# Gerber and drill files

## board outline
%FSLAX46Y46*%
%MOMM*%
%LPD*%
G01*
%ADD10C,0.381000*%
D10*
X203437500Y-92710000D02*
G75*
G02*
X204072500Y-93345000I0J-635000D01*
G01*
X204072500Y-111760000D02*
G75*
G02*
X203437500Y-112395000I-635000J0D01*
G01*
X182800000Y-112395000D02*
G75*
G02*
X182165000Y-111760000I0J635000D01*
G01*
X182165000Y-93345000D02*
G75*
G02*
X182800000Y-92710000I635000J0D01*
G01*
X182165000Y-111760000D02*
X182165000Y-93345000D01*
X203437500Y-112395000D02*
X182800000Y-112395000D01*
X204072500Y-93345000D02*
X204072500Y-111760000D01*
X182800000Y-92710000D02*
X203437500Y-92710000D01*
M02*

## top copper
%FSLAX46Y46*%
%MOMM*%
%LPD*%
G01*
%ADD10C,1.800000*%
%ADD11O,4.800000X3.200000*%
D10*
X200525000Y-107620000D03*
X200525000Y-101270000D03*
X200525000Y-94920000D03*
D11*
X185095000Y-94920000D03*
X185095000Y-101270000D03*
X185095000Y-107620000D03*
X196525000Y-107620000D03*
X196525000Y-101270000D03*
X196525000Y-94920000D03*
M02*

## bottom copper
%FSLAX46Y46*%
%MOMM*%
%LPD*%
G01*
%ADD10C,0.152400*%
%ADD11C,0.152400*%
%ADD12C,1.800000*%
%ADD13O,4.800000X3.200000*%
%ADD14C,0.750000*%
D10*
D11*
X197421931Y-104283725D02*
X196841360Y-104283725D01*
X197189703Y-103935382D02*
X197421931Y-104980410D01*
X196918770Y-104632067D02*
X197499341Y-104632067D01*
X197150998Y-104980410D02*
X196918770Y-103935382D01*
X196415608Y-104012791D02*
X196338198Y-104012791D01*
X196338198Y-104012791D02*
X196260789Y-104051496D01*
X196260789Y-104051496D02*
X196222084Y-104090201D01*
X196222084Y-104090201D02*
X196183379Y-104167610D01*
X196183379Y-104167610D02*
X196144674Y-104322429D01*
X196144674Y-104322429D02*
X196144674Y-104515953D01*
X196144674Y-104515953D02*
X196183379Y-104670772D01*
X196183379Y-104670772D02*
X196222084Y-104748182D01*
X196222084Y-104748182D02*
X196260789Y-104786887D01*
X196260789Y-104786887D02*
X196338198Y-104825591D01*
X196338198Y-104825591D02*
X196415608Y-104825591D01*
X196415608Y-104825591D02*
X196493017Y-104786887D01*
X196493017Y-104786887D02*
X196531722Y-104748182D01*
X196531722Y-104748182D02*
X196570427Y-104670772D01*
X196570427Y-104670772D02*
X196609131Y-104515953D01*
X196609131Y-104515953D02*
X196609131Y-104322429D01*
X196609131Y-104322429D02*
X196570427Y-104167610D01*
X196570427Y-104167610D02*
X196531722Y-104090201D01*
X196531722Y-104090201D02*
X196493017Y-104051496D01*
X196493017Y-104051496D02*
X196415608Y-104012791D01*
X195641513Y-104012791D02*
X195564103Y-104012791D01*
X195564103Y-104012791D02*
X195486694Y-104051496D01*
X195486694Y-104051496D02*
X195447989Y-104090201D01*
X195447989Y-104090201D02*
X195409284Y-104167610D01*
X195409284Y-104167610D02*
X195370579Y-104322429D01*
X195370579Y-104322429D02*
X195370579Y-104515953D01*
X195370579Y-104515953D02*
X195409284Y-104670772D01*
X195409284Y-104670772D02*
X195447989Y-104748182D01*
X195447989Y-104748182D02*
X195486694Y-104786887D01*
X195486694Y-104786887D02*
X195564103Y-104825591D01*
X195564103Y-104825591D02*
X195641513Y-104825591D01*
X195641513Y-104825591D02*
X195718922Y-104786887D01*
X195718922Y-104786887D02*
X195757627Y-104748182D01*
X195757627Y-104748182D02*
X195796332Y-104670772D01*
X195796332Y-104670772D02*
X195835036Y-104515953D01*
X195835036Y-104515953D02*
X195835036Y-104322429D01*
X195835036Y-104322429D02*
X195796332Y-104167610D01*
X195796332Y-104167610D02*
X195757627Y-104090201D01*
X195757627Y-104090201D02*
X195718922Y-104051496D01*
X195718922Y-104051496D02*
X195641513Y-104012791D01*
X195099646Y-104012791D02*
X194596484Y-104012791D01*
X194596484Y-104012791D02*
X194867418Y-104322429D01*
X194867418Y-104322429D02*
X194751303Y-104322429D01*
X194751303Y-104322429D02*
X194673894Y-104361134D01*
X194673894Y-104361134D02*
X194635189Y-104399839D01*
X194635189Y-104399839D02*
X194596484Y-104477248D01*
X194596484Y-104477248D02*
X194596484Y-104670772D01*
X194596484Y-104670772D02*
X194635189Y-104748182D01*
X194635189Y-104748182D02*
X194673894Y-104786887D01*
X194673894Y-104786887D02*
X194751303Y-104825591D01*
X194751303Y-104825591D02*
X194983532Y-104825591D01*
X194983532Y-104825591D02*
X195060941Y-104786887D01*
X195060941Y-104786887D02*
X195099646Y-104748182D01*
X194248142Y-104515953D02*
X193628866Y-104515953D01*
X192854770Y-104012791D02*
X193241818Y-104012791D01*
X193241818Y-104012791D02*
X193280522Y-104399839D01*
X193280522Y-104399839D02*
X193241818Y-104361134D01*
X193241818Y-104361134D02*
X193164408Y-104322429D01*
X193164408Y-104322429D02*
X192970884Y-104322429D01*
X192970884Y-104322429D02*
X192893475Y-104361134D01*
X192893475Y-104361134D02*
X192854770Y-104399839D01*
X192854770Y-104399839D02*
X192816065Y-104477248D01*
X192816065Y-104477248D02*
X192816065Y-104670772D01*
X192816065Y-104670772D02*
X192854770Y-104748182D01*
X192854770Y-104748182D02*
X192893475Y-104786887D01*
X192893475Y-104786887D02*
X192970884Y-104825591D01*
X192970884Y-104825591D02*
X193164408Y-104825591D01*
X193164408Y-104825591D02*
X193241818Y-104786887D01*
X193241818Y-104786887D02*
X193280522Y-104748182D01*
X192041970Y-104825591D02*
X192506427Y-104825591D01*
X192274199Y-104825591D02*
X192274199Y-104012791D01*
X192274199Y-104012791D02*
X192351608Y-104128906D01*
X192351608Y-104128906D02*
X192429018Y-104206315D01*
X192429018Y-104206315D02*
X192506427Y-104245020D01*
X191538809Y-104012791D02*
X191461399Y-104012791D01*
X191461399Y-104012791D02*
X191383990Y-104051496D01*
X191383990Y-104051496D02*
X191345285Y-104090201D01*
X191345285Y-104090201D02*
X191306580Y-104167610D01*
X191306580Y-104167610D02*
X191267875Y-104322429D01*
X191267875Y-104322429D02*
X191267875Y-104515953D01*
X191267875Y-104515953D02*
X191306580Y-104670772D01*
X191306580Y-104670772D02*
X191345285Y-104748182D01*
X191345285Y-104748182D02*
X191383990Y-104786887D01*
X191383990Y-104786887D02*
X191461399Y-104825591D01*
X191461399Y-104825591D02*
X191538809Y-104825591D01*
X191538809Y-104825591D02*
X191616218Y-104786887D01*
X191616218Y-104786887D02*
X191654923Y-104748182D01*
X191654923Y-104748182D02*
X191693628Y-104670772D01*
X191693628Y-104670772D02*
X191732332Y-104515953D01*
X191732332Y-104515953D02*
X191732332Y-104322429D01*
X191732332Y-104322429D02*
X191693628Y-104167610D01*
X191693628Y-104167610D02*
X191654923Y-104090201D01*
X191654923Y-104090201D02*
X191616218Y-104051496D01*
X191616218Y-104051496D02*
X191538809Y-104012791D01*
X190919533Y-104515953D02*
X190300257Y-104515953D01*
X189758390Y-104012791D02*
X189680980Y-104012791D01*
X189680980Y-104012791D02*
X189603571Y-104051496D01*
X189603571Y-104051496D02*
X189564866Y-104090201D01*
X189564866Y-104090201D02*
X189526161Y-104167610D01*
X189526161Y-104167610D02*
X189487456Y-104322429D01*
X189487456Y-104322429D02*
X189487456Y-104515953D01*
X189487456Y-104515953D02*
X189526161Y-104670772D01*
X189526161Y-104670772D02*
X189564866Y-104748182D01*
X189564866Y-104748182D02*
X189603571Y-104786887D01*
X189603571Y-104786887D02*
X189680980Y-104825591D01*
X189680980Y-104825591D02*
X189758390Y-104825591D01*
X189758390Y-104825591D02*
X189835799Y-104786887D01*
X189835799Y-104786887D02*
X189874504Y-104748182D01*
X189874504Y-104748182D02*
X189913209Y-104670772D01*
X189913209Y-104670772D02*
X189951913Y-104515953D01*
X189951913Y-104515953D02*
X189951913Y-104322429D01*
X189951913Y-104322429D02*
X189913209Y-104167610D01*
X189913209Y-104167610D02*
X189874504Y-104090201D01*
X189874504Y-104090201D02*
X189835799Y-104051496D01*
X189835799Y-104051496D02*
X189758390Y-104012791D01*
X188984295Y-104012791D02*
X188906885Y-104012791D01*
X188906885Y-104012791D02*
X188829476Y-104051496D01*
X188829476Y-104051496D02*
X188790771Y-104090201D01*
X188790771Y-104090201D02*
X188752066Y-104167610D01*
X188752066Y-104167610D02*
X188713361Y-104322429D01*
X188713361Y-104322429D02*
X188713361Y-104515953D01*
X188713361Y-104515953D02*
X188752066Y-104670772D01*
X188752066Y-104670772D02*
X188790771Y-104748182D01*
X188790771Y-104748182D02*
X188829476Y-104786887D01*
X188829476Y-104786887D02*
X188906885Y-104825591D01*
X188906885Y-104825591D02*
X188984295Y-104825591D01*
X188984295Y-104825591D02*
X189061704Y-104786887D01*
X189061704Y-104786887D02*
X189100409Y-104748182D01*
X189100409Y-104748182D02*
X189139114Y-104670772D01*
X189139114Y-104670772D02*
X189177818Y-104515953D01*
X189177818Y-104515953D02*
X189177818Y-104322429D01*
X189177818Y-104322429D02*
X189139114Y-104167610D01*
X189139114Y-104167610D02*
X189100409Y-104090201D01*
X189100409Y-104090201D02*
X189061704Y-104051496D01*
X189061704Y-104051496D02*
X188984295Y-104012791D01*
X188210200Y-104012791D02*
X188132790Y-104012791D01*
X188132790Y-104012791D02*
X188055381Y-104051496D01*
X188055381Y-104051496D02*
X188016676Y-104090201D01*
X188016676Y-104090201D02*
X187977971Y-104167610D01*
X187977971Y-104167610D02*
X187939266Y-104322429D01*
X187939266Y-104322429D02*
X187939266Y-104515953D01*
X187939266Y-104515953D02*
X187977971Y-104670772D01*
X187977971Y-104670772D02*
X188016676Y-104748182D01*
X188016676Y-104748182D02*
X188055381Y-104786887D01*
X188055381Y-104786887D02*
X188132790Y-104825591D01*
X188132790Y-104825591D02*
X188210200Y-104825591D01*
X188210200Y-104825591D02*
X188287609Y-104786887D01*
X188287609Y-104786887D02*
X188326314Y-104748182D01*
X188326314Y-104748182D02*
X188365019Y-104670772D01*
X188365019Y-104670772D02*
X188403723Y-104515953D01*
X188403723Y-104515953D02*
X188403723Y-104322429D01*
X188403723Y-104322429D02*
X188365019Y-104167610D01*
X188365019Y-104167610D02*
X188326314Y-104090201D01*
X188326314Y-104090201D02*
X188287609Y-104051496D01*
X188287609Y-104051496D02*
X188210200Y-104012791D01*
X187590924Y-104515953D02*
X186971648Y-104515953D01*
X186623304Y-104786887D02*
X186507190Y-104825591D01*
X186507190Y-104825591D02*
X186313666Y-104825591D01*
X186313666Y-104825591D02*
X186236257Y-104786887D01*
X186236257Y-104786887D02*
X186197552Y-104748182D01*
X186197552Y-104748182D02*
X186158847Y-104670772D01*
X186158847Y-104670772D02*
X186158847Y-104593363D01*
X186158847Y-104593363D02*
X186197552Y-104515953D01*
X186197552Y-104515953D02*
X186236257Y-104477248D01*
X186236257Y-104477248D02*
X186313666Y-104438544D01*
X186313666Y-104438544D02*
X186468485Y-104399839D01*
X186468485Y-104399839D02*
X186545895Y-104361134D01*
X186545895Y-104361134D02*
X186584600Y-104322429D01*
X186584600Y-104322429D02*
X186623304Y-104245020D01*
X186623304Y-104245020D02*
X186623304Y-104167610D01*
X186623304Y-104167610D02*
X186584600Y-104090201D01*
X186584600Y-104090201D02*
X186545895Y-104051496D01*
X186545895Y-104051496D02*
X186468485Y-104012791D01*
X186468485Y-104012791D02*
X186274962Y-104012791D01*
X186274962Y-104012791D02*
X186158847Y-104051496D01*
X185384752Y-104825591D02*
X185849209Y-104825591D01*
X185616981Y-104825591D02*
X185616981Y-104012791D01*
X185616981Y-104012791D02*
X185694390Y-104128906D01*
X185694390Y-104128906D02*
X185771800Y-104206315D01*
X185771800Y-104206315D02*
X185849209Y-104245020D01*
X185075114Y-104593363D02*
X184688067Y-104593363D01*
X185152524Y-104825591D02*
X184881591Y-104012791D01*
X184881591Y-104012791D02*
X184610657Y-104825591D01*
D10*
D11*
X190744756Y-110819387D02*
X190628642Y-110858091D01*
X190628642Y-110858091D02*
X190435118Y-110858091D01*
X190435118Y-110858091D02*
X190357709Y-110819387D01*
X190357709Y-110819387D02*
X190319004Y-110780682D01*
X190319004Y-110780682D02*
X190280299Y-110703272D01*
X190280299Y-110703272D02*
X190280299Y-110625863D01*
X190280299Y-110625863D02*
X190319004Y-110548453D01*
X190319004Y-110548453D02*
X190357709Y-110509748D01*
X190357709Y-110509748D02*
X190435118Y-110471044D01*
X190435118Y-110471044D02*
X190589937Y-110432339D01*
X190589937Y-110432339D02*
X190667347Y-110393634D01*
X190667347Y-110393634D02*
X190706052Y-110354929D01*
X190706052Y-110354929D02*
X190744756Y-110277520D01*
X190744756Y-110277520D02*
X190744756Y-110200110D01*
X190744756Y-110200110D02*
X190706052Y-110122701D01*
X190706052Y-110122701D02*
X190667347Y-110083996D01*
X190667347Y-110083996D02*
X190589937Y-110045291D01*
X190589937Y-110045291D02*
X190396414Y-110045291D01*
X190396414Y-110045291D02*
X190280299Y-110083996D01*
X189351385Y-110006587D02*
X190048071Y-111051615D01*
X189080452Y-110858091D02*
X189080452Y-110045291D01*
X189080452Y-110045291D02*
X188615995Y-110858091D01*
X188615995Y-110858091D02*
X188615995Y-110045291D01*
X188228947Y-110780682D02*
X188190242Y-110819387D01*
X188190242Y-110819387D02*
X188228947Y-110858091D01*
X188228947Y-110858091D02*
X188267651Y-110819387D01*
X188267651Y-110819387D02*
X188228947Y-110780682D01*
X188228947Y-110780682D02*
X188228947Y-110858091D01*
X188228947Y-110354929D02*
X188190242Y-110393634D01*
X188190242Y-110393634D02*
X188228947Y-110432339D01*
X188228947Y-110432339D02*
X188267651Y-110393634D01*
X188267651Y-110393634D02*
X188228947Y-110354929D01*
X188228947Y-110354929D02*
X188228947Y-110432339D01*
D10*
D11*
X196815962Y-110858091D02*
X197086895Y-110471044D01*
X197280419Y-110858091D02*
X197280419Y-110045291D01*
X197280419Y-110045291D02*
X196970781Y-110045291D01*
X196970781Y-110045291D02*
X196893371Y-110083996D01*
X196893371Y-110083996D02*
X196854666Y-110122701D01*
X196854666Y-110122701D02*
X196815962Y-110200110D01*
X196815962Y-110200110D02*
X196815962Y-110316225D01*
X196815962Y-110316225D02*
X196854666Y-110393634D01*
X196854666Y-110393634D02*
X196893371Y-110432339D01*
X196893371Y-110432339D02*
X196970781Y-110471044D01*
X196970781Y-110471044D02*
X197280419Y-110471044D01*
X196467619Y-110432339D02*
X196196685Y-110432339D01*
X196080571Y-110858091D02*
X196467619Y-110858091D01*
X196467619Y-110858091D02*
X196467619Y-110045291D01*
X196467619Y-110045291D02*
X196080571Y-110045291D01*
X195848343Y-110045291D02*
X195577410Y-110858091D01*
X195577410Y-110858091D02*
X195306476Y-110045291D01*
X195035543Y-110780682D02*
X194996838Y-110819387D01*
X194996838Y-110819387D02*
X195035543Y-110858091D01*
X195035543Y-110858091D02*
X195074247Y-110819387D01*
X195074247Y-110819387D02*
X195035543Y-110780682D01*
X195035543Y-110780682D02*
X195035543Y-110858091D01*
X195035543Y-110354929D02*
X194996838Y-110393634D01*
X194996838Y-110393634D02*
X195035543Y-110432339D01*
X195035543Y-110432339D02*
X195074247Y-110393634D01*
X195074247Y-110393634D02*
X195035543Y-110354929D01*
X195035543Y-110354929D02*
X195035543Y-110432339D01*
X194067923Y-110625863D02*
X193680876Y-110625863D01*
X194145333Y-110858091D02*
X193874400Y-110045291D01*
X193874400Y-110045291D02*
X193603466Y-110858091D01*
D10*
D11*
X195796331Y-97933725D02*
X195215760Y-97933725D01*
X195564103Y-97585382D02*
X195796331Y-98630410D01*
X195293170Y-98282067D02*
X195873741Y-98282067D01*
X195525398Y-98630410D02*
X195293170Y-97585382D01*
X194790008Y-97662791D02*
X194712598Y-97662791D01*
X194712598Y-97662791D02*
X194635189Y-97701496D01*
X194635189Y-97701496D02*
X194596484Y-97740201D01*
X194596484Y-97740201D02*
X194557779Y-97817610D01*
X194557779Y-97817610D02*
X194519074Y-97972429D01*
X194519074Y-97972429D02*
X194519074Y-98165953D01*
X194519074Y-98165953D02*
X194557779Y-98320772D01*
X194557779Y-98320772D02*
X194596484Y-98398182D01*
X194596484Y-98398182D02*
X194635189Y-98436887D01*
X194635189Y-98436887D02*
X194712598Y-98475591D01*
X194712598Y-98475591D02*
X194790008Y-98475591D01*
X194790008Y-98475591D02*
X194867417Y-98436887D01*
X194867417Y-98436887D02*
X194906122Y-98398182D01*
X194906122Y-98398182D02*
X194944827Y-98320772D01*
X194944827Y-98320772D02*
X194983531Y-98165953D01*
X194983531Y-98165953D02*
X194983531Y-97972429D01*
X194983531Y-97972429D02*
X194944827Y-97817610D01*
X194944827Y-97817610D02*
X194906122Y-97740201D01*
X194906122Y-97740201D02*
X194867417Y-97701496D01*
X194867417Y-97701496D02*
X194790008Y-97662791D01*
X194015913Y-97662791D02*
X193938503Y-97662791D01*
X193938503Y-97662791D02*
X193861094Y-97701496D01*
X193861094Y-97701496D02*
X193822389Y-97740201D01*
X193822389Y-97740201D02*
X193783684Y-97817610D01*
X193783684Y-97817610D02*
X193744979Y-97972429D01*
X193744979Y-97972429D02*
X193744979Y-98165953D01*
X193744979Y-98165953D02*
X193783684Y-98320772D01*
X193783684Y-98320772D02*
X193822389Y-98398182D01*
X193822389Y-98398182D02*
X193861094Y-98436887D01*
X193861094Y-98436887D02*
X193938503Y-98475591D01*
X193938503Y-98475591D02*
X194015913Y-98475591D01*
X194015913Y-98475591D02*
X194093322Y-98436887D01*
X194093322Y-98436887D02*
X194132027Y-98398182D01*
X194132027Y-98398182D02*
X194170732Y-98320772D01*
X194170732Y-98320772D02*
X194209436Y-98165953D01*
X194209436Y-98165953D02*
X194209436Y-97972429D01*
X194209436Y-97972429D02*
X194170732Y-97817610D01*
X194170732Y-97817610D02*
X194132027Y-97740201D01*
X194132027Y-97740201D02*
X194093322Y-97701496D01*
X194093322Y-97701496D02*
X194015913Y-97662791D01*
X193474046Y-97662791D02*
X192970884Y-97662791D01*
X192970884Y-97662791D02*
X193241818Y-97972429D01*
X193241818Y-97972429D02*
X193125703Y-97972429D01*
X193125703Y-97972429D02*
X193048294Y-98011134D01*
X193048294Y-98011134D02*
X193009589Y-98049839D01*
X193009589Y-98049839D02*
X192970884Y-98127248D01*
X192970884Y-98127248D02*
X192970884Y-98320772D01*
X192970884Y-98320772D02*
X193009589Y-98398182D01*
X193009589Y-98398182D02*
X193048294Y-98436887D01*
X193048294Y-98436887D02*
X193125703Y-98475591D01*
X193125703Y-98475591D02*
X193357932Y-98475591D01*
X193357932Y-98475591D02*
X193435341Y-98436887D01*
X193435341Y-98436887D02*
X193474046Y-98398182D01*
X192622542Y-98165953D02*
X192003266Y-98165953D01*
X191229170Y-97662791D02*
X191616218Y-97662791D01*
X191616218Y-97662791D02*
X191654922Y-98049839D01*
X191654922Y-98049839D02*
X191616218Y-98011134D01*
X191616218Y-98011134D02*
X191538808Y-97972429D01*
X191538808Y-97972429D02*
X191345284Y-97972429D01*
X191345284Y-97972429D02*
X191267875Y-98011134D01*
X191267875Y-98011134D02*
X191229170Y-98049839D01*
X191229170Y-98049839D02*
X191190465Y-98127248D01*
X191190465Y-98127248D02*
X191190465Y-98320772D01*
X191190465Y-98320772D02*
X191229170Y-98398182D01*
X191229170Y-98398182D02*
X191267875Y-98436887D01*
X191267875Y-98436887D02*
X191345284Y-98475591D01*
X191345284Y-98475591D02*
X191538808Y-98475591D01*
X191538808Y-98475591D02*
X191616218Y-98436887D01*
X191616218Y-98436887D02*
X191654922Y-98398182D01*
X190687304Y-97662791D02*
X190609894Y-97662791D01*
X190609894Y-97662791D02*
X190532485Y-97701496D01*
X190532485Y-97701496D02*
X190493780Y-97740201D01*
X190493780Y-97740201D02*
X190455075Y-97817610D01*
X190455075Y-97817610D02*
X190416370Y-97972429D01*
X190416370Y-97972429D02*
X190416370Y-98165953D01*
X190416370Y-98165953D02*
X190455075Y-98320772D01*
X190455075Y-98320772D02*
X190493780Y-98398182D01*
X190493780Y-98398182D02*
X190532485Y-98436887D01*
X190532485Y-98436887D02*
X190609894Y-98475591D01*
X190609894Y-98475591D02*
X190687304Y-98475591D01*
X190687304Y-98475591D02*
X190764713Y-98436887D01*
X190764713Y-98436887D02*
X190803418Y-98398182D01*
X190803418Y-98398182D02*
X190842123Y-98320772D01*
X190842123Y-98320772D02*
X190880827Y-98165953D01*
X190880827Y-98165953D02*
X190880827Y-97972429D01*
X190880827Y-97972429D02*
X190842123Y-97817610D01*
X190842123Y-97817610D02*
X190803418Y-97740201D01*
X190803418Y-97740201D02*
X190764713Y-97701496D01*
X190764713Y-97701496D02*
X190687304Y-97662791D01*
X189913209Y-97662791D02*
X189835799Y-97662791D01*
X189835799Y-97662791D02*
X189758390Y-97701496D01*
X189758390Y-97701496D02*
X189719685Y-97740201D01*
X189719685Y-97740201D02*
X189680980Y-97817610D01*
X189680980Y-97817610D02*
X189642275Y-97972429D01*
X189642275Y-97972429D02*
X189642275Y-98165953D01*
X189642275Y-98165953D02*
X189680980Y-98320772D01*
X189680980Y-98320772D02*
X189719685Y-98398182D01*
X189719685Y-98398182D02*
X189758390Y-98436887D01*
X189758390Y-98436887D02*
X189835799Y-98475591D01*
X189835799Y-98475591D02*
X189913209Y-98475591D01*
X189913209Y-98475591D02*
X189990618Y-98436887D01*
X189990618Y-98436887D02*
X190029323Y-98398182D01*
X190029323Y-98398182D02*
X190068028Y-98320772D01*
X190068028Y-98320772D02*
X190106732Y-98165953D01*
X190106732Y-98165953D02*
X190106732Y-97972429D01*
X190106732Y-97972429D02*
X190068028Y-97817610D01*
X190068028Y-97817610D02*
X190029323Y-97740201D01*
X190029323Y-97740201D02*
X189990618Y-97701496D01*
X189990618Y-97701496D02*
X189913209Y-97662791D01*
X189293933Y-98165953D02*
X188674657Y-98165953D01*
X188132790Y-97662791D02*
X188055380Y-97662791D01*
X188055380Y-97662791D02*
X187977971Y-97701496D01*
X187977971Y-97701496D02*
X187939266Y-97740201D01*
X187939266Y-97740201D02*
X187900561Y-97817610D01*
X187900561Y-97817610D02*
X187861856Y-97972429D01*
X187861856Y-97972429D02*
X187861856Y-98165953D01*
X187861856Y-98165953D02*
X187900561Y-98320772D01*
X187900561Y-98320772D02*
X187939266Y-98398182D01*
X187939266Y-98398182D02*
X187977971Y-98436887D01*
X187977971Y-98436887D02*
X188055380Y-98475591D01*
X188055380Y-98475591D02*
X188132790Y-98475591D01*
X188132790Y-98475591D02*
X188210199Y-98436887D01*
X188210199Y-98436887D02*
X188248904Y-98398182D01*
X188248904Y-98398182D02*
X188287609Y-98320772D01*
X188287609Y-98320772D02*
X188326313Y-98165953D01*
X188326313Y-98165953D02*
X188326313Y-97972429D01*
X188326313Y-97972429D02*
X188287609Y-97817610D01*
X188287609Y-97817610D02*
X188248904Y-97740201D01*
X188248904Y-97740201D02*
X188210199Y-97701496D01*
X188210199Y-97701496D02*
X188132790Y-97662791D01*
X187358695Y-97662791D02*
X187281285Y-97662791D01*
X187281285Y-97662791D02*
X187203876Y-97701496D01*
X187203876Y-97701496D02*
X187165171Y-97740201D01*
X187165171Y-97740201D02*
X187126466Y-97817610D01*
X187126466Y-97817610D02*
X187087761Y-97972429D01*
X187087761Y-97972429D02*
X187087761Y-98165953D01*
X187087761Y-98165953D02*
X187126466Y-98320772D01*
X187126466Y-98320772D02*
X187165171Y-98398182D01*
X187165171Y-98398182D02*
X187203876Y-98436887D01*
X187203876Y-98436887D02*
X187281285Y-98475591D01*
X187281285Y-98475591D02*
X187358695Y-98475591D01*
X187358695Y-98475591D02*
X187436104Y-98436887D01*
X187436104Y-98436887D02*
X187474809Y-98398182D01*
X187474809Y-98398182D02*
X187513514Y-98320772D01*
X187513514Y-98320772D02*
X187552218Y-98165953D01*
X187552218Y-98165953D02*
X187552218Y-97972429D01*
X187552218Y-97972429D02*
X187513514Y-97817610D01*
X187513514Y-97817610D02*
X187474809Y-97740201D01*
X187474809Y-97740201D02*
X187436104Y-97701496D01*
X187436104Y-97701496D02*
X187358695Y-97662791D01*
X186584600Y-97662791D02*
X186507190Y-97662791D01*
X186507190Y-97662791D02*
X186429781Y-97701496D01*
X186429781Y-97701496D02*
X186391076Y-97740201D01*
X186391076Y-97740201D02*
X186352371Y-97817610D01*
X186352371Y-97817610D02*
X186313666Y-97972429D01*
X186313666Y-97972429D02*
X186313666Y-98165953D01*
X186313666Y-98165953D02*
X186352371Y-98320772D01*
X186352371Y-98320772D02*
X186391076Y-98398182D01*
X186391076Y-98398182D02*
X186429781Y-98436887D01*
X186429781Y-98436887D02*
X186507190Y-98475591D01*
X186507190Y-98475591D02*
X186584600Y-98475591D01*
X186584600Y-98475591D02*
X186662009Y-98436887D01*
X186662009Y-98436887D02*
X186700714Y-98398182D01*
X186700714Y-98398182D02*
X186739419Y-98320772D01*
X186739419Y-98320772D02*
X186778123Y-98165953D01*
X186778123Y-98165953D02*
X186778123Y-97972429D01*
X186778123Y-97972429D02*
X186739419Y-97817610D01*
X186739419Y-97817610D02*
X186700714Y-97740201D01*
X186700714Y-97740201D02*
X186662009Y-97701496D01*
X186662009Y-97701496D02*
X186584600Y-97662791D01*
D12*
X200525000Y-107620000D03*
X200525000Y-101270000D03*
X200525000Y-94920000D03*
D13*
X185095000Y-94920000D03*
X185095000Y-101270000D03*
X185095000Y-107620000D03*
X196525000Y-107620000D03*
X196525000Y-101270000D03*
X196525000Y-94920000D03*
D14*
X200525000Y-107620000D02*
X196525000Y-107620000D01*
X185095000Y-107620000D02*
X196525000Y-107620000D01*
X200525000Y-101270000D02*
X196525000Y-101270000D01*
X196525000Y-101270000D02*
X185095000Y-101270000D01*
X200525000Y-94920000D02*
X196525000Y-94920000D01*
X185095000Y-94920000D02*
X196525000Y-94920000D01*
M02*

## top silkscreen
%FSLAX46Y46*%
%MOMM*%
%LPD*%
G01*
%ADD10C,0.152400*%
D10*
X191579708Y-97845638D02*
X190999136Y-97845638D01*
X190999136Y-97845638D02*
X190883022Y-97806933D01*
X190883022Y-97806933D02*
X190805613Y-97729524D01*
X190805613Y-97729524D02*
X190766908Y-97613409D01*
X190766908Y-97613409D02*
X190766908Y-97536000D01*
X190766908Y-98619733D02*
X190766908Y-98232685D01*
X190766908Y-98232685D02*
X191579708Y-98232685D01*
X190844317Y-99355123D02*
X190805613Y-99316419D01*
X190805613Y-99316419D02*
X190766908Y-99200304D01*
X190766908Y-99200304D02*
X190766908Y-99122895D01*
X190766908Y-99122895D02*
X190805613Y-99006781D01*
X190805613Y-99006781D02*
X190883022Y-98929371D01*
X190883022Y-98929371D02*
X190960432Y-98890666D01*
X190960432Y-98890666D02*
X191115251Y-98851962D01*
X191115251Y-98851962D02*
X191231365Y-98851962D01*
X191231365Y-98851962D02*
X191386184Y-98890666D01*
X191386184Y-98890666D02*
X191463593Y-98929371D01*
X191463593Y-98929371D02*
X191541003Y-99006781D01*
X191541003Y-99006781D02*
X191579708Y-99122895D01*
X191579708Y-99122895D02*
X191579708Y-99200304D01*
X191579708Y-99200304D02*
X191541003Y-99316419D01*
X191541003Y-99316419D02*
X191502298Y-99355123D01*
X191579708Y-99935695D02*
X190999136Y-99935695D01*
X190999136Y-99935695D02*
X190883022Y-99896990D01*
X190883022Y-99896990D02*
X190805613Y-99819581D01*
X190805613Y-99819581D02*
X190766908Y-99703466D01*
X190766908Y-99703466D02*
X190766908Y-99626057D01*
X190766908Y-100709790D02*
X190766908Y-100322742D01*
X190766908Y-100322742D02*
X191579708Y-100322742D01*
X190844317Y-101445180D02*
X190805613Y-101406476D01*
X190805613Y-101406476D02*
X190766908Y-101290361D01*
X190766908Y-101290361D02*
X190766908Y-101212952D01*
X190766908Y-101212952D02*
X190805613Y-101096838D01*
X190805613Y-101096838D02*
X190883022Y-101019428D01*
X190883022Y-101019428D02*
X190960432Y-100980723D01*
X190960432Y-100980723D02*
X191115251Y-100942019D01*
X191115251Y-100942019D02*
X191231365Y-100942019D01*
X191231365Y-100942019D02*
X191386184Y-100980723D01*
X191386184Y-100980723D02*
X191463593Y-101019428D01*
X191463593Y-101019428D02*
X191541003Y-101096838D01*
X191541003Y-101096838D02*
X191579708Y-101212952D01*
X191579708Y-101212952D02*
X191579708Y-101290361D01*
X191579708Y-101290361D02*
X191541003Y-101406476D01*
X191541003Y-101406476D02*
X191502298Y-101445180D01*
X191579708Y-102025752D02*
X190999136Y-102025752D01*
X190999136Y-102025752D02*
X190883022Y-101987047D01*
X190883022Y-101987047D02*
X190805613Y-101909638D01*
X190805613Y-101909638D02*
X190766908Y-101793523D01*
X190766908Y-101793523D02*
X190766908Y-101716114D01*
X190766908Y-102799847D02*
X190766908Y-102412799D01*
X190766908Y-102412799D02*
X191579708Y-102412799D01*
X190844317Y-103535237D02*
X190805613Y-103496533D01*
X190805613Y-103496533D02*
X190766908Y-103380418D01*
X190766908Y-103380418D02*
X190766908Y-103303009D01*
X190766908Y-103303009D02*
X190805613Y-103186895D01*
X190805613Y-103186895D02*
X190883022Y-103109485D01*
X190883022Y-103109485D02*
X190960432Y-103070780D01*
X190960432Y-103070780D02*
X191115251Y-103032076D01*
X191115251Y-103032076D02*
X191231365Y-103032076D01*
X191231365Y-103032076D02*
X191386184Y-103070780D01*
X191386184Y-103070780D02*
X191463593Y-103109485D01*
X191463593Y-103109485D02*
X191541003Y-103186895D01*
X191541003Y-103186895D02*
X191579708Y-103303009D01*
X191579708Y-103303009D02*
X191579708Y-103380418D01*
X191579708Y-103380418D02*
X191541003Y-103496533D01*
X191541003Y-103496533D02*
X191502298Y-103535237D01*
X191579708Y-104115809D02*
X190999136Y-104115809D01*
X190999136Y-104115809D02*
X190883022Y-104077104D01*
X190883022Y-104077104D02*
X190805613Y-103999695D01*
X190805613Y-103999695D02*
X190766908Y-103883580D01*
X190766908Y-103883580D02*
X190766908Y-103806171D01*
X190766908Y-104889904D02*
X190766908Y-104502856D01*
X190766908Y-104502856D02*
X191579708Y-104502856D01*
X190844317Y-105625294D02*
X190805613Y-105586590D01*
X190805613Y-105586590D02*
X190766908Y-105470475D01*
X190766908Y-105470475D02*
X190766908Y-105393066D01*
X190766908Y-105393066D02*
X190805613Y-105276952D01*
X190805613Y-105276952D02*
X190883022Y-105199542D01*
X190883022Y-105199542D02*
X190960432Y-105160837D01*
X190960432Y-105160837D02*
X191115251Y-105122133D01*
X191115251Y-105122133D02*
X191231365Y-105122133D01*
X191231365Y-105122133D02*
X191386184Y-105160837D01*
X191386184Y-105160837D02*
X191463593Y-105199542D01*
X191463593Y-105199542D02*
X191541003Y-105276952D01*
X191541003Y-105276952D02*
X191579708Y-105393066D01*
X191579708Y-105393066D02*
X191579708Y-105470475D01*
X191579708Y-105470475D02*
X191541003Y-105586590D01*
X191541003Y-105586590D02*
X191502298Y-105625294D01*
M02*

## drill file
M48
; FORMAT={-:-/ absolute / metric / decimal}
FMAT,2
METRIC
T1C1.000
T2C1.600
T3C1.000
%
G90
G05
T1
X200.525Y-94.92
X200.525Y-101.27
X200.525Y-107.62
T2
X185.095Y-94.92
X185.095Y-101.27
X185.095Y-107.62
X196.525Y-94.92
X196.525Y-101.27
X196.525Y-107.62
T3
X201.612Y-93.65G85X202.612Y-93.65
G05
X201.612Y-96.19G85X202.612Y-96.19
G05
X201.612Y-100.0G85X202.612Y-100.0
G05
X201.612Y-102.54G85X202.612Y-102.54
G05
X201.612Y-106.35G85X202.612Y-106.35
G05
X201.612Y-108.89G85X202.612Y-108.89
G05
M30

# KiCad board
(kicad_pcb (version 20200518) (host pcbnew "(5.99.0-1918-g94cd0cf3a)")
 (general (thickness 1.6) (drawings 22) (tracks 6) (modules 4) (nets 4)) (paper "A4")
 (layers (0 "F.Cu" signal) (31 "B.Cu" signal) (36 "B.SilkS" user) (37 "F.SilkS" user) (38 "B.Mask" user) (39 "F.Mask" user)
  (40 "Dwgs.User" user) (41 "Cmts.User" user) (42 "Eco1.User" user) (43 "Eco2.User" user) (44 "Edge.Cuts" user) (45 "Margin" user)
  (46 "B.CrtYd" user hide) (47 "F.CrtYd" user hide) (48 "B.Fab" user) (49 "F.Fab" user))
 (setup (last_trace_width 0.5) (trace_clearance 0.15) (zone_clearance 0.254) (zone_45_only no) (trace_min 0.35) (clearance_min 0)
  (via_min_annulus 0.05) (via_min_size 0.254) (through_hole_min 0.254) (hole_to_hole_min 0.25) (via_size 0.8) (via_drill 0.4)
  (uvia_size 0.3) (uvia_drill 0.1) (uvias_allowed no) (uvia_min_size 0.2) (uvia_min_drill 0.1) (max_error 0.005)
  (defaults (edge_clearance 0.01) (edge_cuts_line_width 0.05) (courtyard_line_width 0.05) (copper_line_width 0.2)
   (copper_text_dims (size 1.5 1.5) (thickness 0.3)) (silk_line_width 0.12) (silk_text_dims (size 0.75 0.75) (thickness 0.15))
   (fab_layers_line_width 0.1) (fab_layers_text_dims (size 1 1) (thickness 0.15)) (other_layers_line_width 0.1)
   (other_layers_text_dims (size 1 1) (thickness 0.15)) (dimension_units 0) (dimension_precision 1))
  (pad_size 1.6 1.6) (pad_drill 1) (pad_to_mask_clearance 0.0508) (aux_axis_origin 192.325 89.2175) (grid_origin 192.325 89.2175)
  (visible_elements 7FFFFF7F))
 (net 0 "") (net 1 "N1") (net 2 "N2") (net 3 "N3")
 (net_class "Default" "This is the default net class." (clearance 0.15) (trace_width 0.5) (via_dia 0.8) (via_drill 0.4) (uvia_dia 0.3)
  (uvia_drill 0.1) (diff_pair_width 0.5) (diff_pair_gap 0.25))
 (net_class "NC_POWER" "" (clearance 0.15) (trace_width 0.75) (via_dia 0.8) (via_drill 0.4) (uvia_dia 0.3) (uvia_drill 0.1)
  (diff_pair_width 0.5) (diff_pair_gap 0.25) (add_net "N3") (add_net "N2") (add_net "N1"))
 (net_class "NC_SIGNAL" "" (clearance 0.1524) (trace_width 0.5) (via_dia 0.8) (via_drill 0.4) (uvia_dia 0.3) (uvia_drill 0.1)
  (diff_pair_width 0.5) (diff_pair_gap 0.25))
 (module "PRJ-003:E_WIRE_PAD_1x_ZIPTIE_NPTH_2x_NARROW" (layer "F.Cu") (at 200.525 107.62)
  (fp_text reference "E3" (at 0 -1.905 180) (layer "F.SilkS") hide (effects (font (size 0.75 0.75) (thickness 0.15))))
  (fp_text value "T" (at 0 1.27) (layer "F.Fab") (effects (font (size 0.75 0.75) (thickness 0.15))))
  (pad "" np_thru_hole oval (at 1.5875 1.27 90) (size 1 2) (drill oval 1 2) (layers *.Cu *.Mask))
  (pad "" np_thru_hole oval (at 1.5875 -1.27 90) (size 1 2) (drill oval 1 2) (layers *.Cu *.Mask))
  (pad "" connect circle (at 0 0) (size 1 1) (layers "F.Mask"))
  (pad "1" thru_hole circle (at 0 0) (size 1.8 1.8) (drill 1) (layers "B.Cu" "B.Mask") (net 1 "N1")))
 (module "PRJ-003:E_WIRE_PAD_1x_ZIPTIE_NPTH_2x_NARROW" (layer "F.Cu") (at 200.525 101.27)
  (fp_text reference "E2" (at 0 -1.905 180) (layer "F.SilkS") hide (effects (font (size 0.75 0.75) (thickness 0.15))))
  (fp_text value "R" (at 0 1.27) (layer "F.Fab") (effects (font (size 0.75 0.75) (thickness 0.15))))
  (pad "" np_thru_hole oval (at 1.5875 1.27 90) (size 1 2) (drill oval 1 2) (layers *.Cu *.Mask))
  (pad "" np_thru_hole oval (at 1.5875 -1.27 90) (size 1 2) (drill oval 1 2) (layers *.Cu *.Mask))
  (pad "" connect circle (at 0 0) (size 1 1) (layers "F.Mask"))
  (pad "1" thru_hole circle (at 0 0) (size 1.8 1.8) (drill 1) (layers "B.Cu" "B.Mask") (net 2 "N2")))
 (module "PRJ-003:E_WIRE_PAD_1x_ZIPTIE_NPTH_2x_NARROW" (layer "F.Cu") (at 200.525 94.92)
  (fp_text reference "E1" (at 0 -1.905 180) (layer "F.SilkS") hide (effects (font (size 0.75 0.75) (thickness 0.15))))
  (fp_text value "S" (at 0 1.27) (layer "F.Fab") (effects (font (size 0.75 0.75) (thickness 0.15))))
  (pad "" np_thru_hole oval (at 1.5875 1.27 90) (size 1 2) (drill oval 1 2) (layers *.Cu *.Mask))
  (pad "" np_thru_hole oval (at 1.5875 -1.27 90) (size 1 2) (drill oval 1 2) (layers *.Cu *.Mask))
  (pad "" connect circle (at 0 0) (size 1 1) (layers "F.Mask"))
  (pad "1" thru_hole circle (at 0 0) (size 1.8 1.8) (drill 1) (layers "B.Cu" "B.Mask") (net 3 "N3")))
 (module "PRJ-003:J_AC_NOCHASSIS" (layer "F.Cu") (at 192.325 90.17)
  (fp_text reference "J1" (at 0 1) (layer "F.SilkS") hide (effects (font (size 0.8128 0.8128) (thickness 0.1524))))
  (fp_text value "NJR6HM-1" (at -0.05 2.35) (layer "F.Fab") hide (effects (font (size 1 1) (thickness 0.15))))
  (pad "" connect circle (at 4.2 4.75) (size 1.6 1.6) (layers "F.Mask"))
  (pad "" connect circle (at 4.2 11.1) (size 1.6 1.6) (layers "F.Mask"))
  (pad "" connect circle (at 4.2 17.45) (size 1.6 1.6) (layers "F.Mask"))
  (pad "" connect circle (at -7.23 17.45) (size 1.6 1.6) (layers "F.Mask"))
  (pad "" connect circle (at -7.23 11.1) (size 1.6 1.6) (layers "F.Mask"))
  (pad "" connect circle (at -7.23 4.75) (size 1.6 1.6) (layers "F.Mask"))
  (pad "S" thru_hole oval (at -7.23 4.75) (size 4.8 3.2) (drill 1.6) (layers "B.Cu" "B.Mask") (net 3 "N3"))
  (pad "R" thru_hole oval (at -7.23 11.1) (size 4.8 3.2) (drill 1.6) (layers "B.Cu" "B.Mask") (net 2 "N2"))
  (pad "T" thru_hole oval (at -7.23 17.45) (size 4.8 3.2) (drill 1.6) (layers "B.Cu" "B.Mask") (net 1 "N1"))
  (pad "TN" thru_hole oval (at 4.2 17.45) (size 4.8 3.2) (drill 1.6) (layers "B.Cu" "B.Mask") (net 1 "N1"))
  (pad "RN" thru_hole oval (at 4.2 11.1) (size 4.8 3.2) (drill 1.6) (layers "B.Cu" "B.Mask") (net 2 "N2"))
  (pad "SN" thru_hole oval (at 4.2 4.75) (size 4.8 3.2) (drill 1.6) (layers "B.Cu" "B.Mask") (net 3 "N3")))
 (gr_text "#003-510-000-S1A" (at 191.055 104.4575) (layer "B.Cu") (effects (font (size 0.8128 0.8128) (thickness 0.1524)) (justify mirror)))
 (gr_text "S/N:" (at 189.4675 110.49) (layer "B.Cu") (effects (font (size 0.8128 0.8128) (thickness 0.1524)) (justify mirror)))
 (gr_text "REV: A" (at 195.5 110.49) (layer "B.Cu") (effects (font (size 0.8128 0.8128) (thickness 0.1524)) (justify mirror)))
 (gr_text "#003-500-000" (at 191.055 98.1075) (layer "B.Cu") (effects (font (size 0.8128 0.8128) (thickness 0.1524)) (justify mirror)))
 (gr_arc (start 203.4375 93.345) (end 204.0725 93.345) (angle -90) (layer "Edge.Cuts") (width 0.381))
 (gr_arc (start 203.4375 111.76) (end 203.4375 112.395) (angle -90) (layer "Edge.Cuts") (width 0.381))
 (gr_arc (start 182.8 111.76) (end 182.165 111.76) (angle -90) (layer "Edge.Cuts") (width 0.381))
 (gr_arc (start 182.8 93.345) (end 182.8 92.71) (angle -90) (layer "Edge.Cuts") (width 0.381))
 (gr_line (start 182.165 111.76) (end 182.165 93.345) (layer "Edge.Cuts") (width 0.381))
 (gr_line (start 203.4375 112.395) (end 182.8 112.395) (layer "Edge.Cuts") (width 0.381))
 (gr_line (start 204.0725 93.345) (end 204.0725 111.76) (layer "Edge.Cuts") (width 0.381))
 (gr_line (start 182.8 92.71) (end 203.4375 92.71) (layer "Edge.Cuts") (width 0.381))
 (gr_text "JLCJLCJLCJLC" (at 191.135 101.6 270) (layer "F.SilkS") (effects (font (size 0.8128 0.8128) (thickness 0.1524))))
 (segment (start 200.525 107.62) (end 196.525 107.62) (width 0.75) (layer "B.Cu") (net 1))
 (segment (start 185.095 107.62) (end 196.525 107.62) (width 0.75) (layer "B.Cu") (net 1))
 (segment (start 200.525 101.27) (end 196.525 101.27) (width 0.75) (layer "B.Cu") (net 2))
 (segment (start 196.525 101.27) (end 185.095 101.27) (width 0.75) (layer "B.Cu") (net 2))
 (segment (start 200.525 94.92) (end 196.525 94.92) (width 0.75) (layer "B.Cu") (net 3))
 (segment (start 185.095 94.92) (end 196.525 94.92) (width 0.75) (layer "B.Cu") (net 3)))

